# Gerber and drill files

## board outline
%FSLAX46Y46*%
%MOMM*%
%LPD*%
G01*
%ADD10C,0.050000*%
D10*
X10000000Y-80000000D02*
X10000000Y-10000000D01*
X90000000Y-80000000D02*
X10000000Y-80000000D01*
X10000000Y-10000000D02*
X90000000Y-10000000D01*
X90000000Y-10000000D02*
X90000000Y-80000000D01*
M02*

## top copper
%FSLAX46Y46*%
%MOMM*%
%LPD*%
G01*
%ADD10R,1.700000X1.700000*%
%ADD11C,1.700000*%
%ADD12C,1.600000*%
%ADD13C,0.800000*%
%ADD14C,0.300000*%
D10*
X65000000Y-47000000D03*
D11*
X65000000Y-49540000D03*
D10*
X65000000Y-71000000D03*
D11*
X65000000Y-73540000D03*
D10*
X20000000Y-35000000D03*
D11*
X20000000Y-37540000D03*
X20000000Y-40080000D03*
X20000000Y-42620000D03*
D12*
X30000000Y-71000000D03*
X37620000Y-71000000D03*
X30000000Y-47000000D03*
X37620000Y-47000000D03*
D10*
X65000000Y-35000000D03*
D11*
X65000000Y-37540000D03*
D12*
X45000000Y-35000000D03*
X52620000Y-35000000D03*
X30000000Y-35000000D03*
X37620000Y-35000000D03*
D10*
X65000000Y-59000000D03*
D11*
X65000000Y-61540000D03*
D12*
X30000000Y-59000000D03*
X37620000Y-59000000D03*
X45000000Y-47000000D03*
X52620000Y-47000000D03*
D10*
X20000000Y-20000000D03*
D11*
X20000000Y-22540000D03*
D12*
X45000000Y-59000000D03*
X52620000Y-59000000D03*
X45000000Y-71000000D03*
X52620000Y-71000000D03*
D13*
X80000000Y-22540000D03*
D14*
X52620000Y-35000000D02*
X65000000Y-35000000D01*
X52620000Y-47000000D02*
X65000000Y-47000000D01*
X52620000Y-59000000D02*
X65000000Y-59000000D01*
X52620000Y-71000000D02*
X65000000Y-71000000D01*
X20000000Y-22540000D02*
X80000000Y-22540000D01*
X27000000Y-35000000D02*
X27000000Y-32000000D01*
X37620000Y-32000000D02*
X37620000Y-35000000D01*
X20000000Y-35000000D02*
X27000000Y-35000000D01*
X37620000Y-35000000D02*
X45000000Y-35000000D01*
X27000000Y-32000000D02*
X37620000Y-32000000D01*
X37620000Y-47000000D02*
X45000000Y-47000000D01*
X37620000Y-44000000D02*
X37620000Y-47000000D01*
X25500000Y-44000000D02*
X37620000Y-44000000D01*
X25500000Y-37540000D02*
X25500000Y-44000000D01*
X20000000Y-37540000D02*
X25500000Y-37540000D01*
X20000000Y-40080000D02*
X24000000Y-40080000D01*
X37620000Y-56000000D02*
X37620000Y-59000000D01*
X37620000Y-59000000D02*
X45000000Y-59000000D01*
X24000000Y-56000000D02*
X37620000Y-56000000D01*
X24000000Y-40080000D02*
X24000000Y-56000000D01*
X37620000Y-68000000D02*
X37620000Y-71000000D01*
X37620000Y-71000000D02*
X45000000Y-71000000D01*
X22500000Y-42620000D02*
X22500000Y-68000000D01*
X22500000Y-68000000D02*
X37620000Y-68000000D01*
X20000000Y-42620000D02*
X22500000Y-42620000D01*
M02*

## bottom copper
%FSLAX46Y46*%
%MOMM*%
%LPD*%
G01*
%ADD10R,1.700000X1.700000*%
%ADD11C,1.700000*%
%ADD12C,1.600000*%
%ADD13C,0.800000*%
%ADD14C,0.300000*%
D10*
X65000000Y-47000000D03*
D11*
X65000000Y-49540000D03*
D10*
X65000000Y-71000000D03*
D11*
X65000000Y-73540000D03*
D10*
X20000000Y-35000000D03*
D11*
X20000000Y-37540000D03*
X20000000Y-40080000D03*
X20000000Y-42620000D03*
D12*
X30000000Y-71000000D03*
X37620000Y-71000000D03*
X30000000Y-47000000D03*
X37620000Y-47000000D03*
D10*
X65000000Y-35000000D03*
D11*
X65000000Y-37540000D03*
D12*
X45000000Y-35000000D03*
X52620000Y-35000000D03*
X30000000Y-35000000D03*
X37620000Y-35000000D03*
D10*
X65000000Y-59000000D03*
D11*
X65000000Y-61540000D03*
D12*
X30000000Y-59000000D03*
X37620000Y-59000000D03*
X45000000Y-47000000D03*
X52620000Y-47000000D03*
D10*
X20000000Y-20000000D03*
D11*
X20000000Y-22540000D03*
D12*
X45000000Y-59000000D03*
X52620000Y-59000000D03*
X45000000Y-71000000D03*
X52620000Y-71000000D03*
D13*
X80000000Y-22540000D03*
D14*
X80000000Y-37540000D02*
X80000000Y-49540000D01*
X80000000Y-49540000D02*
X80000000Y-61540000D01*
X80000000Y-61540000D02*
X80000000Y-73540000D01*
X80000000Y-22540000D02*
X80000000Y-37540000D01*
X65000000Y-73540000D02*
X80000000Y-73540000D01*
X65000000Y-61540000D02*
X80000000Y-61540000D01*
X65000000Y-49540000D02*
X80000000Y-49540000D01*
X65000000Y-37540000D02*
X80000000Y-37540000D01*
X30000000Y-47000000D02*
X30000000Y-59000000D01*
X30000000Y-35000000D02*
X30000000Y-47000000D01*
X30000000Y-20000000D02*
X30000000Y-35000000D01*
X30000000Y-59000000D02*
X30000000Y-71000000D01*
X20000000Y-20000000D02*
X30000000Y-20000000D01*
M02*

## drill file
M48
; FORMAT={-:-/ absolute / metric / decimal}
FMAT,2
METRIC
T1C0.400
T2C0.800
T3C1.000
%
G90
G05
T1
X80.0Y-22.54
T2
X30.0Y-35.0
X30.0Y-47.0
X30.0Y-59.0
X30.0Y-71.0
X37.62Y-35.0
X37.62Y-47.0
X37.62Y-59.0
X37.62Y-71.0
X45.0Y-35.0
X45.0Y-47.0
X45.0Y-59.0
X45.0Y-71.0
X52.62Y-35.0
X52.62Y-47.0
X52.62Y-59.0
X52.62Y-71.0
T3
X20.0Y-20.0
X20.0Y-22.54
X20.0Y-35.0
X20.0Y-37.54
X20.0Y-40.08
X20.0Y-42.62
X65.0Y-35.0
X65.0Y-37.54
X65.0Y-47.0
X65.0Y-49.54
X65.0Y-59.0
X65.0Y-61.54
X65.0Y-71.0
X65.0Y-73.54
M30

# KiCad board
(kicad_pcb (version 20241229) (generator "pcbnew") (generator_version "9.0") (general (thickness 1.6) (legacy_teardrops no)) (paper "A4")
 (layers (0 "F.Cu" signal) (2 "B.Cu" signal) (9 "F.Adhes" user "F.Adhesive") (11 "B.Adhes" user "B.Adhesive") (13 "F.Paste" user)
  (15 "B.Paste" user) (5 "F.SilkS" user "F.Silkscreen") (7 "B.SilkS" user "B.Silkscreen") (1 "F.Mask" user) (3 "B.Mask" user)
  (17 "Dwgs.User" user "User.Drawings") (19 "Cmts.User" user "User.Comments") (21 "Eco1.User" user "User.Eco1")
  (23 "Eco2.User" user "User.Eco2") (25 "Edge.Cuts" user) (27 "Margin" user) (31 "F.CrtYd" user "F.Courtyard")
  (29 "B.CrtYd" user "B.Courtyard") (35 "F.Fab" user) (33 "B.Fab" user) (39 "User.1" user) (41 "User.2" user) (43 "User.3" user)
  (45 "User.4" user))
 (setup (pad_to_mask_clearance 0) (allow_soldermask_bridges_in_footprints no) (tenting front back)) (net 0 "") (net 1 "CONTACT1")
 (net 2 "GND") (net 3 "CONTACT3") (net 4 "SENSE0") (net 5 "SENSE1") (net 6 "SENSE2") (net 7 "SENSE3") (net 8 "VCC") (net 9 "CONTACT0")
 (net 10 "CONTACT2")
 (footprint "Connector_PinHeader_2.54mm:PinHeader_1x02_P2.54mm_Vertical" (layer "F.Cu") (at 65 47)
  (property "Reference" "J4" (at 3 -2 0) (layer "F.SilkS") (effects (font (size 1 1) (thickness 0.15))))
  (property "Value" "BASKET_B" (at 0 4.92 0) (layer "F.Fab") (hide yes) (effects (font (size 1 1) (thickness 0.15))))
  (pad "1" thru_hole rect (at 0 0) (size 1.7 1.7) (drill 1) (layers "*.Cu" "*.Mask") (remove_unused_layers no) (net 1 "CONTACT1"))
  (pad "2" thru_hole circle (at 0 2.54) (size 1.7 1.7) (drill 1) (layers "*.Cu" "*.Mask") (remove_unused_layers no) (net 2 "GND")))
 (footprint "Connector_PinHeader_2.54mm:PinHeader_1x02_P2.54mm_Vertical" (layer "F.Cu") (at 65 71)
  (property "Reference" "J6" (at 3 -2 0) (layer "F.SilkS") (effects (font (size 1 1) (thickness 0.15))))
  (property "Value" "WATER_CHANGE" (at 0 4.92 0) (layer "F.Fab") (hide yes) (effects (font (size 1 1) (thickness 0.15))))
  (pad "1" thru_hole rect (at 0 0) (size 1.7 1.7) (drill 1) (layers "*.Cu" "*.Mask") (remove_unused_layers no) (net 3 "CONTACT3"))
  (pad "2" thru_hole circle (at 0 2.54) (size 1.7 1.7) (drill 1) (layers "*.Cu" "*.Mask") (remove_unused_layers no) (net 2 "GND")))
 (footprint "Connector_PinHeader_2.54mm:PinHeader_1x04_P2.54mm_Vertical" (layer "F.Cu") (at 20 35)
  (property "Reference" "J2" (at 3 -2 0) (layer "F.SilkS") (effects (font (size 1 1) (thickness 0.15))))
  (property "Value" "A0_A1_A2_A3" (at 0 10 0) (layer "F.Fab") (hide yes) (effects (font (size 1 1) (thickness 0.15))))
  (pad "1" thru_hole rect (at 0 0) (size 1.7 1.7) (drill 1) (layers "*.Cu" "*.Mask") (remove_unused_layers no) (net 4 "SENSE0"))
  (pad "2" thru_hole circle (at 0 2.54) (size 1.7 1.7) (drill 1) (layers "*.Cu" "*.Mask") (remove_unused_layers no) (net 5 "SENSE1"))
  (pad "3" thru_hole circle (at 0 5.08) (size 1.7 1.7) (drill 1) (layers "*.Cu" "*.Mask") (remove_unused_layers no) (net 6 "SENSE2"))
  (pad "4" thru_hole circle (at 0 7.62) (size 1.7 1.7) (drill 1) (layers "*.Cu" "*.Mask") (remove_unused_layers no) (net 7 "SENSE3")))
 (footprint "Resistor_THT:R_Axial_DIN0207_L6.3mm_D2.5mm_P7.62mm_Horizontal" (layer "F.Cu") (at 30 71)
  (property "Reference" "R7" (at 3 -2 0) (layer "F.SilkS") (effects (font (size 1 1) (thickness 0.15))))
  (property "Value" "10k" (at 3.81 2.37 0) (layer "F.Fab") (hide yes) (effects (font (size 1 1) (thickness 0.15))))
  (pad "1" thru_hole circle (at 0 0) (size 1.6 1.6) (drill 0.8) (layers "*.Cu" "*.Mask") (remove_unused_layers no) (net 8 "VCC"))
  (pad "2" thru_hole circle (at 7.62 0) (size 1.6 1.6) (drill 0.8) (layers "*.Cu" "*.Mask") (remove_unused_layers no) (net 7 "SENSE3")))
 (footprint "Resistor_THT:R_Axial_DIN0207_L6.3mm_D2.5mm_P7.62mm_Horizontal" (layer "F.Cu") (at 30 47)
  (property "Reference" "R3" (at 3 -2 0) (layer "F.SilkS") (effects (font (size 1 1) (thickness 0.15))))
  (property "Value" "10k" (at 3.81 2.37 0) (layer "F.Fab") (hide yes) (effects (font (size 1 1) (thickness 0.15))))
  (pad "1" thru_hole circle (at 0 0) (size 1.6 1.6) (drill 0.8) (layers "*.Cu" "*.Mask") (remove_unused_layers no) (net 8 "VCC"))
  (pad "2" thru_hole circle (at 7.62 0) (size 1.6 1.6) (drill 0.8) (layers "*.Cu" "*.Mask") (remove_unused_layers no) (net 5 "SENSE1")))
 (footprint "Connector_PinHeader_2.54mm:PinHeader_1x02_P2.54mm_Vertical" (layer "F.Cu") (at 65 35)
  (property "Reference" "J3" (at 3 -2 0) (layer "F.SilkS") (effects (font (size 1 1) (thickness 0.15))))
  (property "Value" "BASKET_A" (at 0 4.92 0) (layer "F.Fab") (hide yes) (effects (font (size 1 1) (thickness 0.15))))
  (pad "1" thru_hole rect (at 0 0) (size 1.7 1.7) (drill 1) (layers "*.Cu" "*.Mask") (remove_unused_layers no) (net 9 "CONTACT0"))
  (pad "2" thru_hole circle (at 0 2.54) (size 1.7 1.7) (drill 1) (layers "*.Cu" "*.Mask") (remove_unused_layers no) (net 2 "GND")))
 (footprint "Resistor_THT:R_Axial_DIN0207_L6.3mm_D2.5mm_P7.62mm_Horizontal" (layer "F.Cu") (at 45 35)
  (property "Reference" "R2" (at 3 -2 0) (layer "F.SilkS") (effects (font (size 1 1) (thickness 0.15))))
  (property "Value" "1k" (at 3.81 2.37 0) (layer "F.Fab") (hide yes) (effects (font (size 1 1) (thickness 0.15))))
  (pad "1" thru_hole circle (at 0 0) (size 1.6 1.6) (drill 0.8) (layers "*.Cu" "*.Mask") (remove_unused_layers no) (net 4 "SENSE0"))
  (pad "2" thru_hole circle (at 7.62 0) (size 1.6 1.6) (drill 0.8) (layers "*.Cu" "*.Mask") (remove_unused_layers no) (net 9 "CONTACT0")))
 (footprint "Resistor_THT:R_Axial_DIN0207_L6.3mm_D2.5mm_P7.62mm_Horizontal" (layer "F.Cu") (at 30 35)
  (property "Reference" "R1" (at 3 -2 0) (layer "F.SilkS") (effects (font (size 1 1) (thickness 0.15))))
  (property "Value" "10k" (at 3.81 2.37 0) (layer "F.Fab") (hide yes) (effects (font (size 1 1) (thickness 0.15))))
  (pad "1" thru_hole circle (at 0 0) (size 1.6 1.6) (drill 0.8) (layers "*.Cu" "*.Mask") (remove_unused_layers no) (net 8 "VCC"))
  (pad "2" thru_hole circle (at 7.62 0) (size 1.6 1.6) (drill 0.8) (layers "*.Cu" "*.Mask") (remove_unused_layers no) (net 4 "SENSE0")))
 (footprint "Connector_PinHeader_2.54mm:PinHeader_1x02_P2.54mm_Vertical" (layer "F.Cu") (at 65 59)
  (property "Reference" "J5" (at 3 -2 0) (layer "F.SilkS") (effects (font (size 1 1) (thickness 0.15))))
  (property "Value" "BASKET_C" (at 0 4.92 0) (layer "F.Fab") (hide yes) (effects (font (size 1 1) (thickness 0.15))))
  (pad "1" thru_hole rect (at 0 0) (size 1.7 1.7) (drill 1) (layers "*.Cu" "*.Mask") (remove_unused_layers no) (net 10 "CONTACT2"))
  (pad "2" thru_hole circle (at 0 2.54) (size 1.7 1.7) (drill 1) (layers "*.Cu" "*.Mask") (remove_unused_layers no) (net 2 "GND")))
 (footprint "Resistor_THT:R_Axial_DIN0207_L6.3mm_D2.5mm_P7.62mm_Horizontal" (layer "F.Cu") (at 30 59)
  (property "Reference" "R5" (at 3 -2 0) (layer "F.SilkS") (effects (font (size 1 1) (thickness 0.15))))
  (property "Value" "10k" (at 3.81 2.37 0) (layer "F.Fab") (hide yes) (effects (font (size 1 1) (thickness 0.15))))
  (pad "1" thru_hole circle (at 0 0) (size 1.6 1.6) (drill 0.8) (layers "*.Cu" "*.Mask") (remove_unused_layers no) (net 8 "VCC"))
  (pad "2" thru_hole circle (at 7.62 0) (size 1.6 1.6) (drill 0.8) (layers "*.Cu" "*.Mask") (remove_unused_layers no) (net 6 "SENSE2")))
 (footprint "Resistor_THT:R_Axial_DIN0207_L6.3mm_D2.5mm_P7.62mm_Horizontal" (layer "F.Cu") (at 45 47)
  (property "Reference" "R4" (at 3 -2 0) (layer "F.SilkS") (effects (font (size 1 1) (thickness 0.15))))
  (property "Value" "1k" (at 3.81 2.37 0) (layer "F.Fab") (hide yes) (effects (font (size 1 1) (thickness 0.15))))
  (pad "1" thru_hole circle (at 0 0) (size 1.6 1.6) (drill 0.8) (layers "*.Cu" "*.Mask") (remove_unused_layers no) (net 5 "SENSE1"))
  (pad "2" thru_hole circle (at 7.62 0) (size 1.6 1.6) (drill 0.8) (layers "*.Cu" "*.Mask") (remove_unused_layers no) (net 1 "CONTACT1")))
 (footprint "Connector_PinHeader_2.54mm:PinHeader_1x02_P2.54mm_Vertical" (layer "F.Cu") (at 20 20)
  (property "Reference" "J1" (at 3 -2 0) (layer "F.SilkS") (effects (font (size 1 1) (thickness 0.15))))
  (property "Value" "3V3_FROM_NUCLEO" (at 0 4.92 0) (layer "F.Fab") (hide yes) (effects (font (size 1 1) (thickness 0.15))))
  (pad "1" thru_hole rect (at 0 0) (size 1.7 1.7) (drill 1) (layers "*.Cu" "*.Mask") (remove_unused_layers no) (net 8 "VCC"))
  (pad "2" thru_hole circle (at 0 2.54) (size 1.7 1.7) (drill 1) (layers "*.Cu" "*.Mask") (remove_unused_layers no) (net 2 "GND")))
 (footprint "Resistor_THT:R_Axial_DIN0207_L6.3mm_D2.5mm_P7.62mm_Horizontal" (layer "F.Cu") (at 45 59)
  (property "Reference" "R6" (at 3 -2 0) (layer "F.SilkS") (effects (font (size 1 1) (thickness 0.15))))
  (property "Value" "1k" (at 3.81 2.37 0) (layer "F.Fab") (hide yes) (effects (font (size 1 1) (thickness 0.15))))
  (pad "1" thru_hole circle (at 0 0) (size 1.6 1.6) (drill 0.8) (layers "*.Cu" "*.Mask") (remove_unused_layers no) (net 6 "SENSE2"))
  (pad "2" thru_hole circle (at 7.62 0) (size 1.6 1.6) (drill 0.8) (layers "*.Cu" "*.Mask") (remove_unused_layers no) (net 10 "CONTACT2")))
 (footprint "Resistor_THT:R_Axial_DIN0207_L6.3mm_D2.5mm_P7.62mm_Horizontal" (layer "F.Cu") (at 45 71)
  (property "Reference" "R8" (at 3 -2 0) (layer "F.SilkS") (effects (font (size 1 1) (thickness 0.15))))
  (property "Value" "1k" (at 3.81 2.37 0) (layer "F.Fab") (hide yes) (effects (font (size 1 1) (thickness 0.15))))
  (pad "1" thru_hole circle (at 0 0) (size 1.6 1.6) (drill 0.8) (layers "*.Cu" "*.Mask") (remove_unused_layers no) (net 7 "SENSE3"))
  (pad "2" thru_hole circle (at 7.62 0) (size 1.6 1.6) (drill 0.8) (layers "*.Cu" "*.Mask") (remove_unused_layers no) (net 3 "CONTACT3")))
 (gr_line (start 10 80) (end 10 10) (stroke (width 0.05) (type default)) (layer "Edge.Cuts"))
 (gr_line (start 90 80) (end 10 80) (stroke (width 0.05) (type default)) (layer "Edge.Cuts"))
 (gr_line (start 10 10) (end 90 10) (stroke (width 0.05) (type default)) (layer "Edge.Cuts"))
 (gr_line (start 90 10) (end 90 80) (stroke (width 0.05) (type default)) (layer "Edge.Cuts"))
 (segment (start 52.62 35) (end 65 35) (width 0.3) (layer "F.Cu") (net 9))
 (segment (start 52.62 47) (end 65 47) (width 0.3) (layer "F.Cu") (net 1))
 (segment (start 52.62 59) (end 65 59) (width 0.3) (layer "F.Cu") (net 10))
 (segment (start 52.62 71) (end 65 71) (width 0.3) (layer "F.Cu") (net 3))
 (segment (start 20 22.54) (end 80 22.54) (width 0.3) (layer "F.Cu") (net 2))
 (via (at 80 22.54) (size 0.8) (drill 0.4) (layers "F.Cu" "B.Cu") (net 2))
 (segment (start 80 37.54) (end 80 49.54) (width 0.3) (layer "B.Cu") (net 2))
 (segment (start 80 49.54) (end 80 61.54) (width 0.3) (layer "B.Cu") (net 2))
 (segment (start 80 61.54) (end 80 73.54) (width 0.3) (layer "B.Cu") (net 2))
 (segment (start 80 22.54) (end 80 37.54) (width 0.3) (layer "B.Cu") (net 2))
 (segment (start 65 73.54) (end 80 73.54) (width 0.3) (layer "B.Cu") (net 2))
 (segment (start 65 61.54) (end 80 61.54) (width 0.3) (layer "B.Cu") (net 2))
 (segment (start 65 49.54) (end 80 49.54) (width 0.3) (layer "B.Cu") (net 2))
 (segment (start 65 37.54) (end 80 37.54) (width 0.3) (layer "B.Cu") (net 2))
 (segment (start 27 35) (end 27 32) (width 0.3) (layer "F.Cu") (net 4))
 (segment (start 37.62 32) (end 37.62 35) (width 0.3) (layer "F.Cu") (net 4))
 (segment (start 20 35) (end 27 35) (width 0.3) (layer "F.Cu") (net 4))
 (segment (start 37.62 35) (end 45 35) (width 0.3) (layer "F.Cu") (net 4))
 (segment (start 27 32) (end 37.62 32) (width 0.3) (layer "F.Cu") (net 4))
 (segment (start 37.62 47) (end 45 47) (width 0.3) (layer "F.Cu") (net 5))
 (segment (start 37.62 44) (end 37.62 47) (width 0.3) (layer "F.Cu") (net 5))
 (segment (start 25.5 44) (end 37.62 44) (width 0.3) (layer "F.Cu") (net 5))
 (segment (start 25.5 37.54) (end 25.5 44) (width 0.3) (layer "F.Cu") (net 5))
 (segment (start 20 37.54) (end 25.5 37.54) (width 0.3) (layer "F.Cu") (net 5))
 (segment (start 20 40.08) (end 24 40.08) (width 0.3) (layer "F.Cu") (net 6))
 (segment (start 37.62 56) (end 37.62 59) (width 0.3) (layer "F.Cu") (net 6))
 (segment (start 37.62 59) (end 45 59) (width 0.3) (layer "F.Cu") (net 6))
 (segment (start 24 56) (end 37.62 56) (width 0.3) (layer "F.Cu") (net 6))
 (segment (start 24 40.08) (end 24 56) (width 0.3) (layer "F.Cu") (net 6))
 (segment (start 37.62 68) (end 37.62 71) (width 0.3) (layer "F.Cu") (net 7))
 (segment (start 37.62 71) (end 45 71) (width 0.3) (layer "F.Cu") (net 7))
 (segment (start 22.5 42.62) (end 22.5 68) (width 0.3) (layer "F.Cu") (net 7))
 (segment (start 22.5 68) (end 37.62 68) (width 0.3) (layer "F.Cu") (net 7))
 (segment (start 20 42.62) (end 22.5 42.62) (width 0.3) (layer "F.Cu") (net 7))
 (segment (start 30 47) (end 30 59) (width 0.3) (layer "B.Cu") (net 8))
 (segment (start 30 35) (end 30 47) (width 0.3) (layer "B.Cu") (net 8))
 (segment (start 30 20) (end 30 35) (width 0.3) (layer "B.Cu") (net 8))
 (segment (start 30 59) (end 30 71) (width 0.3) (layer "B.Cu") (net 8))
 (segment (start 20 20) (end 30 20) (width 0.3) (layer "B.Cu") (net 8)))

